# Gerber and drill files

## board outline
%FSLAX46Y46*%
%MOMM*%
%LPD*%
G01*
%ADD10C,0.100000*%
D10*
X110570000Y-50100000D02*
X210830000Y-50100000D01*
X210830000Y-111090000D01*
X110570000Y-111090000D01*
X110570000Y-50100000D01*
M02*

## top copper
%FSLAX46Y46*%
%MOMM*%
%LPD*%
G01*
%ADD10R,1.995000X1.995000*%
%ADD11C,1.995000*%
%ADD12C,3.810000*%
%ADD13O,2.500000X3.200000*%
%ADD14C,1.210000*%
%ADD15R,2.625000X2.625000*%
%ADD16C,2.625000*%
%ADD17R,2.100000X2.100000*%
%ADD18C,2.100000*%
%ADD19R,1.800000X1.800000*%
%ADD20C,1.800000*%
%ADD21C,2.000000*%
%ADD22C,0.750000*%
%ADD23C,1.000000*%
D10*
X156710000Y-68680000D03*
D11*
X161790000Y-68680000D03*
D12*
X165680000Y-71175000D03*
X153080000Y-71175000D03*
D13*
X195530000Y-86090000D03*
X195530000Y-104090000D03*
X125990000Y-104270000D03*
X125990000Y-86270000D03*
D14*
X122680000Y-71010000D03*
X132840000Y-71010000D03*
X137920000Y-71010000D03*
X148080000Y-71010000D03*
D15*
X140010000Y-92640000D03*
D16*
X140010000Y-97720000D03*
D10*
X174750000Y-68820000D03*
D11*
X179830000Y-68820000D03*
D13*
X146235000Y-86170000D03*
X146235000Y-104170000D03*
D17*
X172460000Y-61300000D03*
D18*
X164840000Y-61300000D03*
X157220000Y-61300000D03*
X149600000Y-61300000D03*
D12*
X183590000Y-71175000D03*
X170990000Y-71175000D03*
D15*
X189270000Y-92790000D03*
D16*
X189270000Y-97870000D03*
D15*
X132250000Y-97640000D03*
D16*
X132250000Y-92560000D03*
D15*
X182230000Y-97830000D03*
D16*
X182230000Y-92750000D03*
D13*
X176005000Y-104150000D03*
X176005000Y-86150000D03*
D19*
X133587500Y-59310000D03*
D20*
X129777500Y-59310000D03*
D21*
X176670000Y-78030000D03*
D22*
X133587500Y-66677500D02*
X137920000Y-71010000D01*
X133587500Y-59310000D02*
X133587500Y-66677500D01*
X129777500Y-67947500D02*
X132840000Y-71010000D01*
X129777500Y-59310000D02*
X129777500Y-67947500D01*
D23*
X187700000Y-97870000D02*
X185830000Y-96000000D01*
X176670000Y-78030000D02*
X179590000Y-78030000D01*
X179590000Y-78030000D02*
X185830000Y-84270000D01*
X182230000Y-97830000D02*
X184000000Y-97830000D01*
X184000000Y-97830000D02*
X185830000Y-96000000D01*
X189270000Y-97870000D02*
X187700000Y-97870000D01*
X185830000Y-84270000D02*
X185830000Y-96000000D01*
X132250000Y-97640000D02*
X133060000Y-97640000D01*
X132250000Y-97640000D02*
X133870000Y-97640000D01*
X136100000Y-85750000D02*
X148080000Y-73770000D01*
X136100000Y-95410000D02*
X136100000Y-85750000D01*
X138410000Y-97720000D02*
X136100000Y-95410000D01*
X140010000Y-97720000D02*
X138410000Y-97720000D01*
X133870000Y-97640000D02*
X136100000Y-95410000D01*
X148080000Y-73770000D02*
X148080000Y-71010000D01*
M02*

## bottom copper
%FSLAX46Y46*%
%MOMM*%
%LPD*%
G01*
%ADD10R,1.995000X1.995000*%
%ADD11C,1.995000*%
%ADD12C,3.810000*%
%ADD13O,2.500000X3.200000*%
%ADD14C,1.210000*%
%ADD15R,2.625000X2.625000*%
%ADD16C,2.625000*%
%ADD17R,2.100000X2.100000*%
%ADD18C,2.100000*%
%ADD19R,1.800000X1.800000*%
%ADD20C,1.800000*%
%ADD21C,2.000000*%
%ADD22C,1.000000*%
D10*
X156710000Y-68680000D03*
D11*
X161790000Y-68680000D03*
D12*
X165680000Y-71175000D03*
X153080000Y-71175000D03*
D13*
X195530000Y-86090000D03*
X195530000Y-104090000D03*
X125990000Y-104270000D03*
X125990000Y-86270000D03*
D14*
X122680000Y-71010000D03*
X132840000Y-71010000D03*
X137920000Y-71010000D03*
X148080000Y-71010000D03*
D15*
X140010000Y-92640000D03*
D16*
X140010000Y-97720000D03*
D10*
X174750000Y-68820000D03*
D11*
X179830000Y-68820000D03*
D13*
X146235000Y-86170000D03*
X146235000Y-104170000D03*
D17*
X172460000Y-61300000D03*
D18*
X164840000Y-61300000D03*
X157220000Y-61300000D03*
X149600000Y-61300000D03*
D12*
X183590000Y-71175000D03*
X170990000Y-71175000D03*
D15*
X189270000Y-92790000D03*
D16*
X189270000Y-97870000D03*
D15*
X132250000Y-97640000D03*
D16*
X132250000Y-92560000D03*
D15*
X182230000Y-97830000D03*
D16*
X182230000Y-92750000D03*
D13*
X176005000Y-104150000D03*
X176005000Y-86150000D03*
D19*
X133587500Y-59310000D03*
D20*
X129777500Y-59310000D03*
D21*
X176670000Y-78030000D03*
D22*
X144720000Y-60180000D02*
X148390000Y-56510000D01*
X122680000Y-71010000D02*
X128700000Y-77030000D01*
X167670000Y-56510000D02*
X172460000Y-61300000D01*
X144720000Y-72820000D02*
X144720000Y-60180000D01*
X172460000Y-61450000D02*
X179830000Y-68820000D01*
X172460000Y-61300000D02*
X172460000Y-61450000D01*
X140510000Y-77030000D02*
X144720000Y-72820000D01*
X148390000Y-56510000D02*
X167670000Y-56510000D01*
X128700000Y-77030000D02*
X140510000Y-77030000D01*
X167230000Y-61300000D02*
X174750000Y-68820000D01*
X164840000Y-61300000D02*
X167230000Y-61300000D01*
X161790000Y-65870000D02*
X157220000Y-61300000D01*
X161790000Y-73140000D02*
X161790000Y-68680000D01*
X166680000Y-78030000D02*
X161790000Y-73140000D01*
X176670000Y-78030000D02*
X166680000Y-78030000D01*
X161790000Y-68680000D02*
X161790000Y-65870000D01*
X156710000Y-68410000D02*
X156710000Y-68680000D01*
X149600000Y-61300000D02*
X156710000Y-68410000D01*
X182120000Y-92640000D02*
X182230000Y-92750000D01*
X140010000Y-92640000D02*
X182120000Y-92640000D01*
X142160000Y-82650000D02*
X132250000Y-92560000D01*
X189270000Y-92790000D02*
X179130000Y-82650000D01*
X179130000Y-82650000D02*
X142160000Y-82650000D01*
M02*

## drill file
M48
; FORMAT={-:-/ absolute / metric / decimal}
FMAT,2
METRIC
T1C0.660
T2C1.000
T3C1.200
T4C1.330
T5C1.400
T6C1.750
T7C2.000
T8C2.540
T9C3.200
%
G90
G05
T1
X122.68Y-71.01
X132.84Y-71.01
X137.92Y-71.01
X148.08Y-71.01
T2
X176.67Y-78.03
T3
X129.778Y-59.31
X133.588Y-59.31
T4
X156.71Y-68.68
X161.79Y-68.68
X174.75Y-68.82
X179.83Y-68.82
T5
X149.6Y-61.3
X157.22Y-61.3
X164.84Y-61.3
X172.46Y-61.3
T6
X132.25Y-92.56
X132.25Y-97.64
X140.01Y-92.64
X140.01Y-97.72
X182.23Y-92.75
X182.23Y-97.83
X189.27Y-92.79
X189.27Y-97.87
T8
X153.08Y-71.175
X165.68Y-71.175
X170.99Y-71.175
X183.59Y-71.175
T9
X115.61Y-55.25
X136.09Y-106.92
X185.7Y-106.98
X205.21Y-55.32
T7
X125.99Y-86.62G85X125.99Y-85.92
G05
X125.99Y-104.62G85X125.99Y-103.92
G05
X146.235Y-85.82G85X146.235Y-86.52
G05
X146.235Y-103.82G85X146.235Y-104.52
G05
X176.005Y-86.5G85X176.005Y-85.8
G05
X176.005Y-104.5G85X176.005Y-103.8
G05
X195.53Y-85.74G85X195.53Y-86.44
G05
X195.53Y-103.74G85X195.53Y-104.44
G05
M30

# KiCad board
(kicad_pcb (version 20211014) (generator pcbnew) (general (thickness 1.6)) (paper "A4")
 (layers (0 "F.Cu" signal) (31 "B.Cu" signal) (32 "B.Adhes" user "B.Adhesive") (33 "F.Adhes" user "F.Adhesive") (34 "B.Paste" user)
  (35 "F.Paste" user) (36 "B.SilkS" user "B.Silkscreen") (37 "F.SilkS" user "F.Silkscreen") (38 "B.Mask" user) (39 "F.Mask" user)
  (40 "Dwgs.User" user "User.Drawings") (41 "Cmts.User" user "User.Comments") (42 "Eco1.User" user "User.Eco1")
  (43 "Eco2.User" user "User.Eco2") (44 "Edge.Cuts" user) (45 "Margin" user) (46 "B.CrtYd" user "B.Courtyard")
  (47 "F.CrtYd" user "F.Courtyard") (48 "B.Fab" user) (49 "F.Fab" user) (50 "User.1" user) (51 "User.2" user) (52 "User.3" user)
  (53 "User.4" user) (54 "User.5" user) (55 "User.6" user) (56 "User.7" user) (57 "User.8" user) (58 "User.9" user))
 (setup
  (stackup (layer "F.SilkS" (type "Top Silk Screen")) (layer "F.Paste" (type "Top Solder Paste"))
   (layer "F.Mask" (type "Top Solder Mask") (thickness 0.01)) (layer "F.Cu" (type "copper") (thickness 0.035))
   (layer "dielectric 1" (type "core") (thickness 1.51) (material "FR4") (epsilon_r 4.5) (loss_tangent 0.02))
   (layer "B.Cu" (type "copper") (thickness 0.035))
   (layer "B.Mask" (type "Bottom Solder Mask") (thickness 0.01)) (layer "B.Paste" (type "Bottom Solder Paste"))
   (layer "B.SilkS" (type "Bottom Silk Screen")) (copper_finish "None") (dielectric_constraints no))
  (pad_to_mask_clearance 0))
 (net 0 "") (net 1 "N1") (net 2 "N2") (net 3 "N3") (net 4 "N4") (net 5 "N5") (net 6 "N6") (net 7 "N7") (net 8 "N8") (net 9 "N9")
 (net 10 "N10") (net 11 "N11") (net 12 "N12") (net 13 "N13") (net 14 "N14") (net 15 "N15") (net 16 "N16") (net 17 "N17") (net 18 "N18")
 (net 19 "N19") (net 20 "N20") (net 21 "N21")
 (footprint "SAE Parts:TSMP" (layer "F.Cu") (at 156.71 68.68)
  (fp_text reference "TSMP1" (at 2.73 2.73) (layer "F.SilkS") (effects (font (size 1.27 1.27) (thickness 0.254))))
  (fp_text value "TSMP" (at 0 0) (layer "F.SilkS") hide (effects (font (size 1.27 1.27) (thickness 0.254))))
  (pad "1" thru_hole rect (at 0 0) (size 1.995 1.995) (drill 1.33) (layers *.Cu *.Mask) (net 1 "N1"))
  (pad "2" thru_hole circle (at 5.08 0) (size 1.995 1.995) (drill 1.33) (layers *.Cu *.Mask) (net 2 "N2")))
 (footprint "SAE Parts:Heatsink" (layer "F.Cu") (at 165.68 71.175 180)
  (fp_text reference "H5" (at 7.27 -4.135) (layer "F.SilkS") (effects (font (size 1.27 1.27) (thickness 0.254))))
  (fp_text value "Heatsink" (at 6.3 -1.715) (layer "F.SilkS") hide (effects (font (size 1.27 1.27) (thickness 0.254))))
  (pad "1" thru_hole circle (at 0 0 180) (size 3.81 3.81) (drill 2.54) (layers *.Cu *.Mask) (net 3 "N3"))
  (pad "2" thru_hole circle (at 12.6 0 180) (size 3.81 3.81) (drill 2.54) (layers *.Cu *.Mask) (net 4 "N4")))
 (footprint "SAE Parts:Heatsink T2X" (layer "F.Cu") (at 201.405 95.19 -90)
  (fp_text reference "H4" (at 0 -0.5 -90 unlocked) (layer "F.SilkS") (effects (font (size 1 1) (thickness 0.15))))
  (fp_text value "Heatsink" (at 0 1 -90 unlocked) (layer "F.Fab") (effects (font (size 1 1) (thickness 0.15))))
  (pad "1" thru_hole oval (at -9.1 5.875 270) (size 3.2 2.5) (drill oval 2.7 2) (layers *.Cu *.Mask) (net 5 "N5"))
  (pad "2" thru_hole oval (at 8.9 5.875 270) (size 3.2 2.5) (drill oval 2.7 2) (layers *.Cu *.Mask) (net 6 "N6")))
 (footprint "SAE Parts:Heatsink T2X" (layer "F.Cu") (at 120.115 95.17 90)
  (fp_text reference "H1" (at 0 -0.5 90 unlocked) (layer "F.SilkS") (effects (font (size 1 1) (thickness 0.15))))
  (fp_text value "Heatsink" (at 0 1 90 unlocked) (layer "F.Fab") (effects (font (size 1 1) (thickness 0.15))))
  (pad "1" thru_hole oval (at -9.1 5.875 90) (size 3.2 2.5) (drill oval 2.7 2) (layers *.Cu *.Mask) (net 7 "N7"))
  (pad "2" thru_hole oval (at 8.9 5.875 90) (size 3.2 2.5) (drill oval 2.7 2) (layers *.Cu *.Mask) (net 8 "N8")))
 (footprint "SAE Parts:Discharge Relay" (layer "F.Cu") (at 122.68 71.01)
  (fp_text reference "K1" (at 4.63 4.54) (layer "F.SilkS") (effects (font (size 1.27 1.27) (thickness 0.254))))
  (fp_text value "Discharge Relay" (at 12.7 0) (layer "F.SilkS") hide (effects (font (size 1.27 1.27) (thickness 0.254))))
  (pad "1" thru_hole circle (at 0 0) (size 1.21 1.21) (drill 0.66) (layers *.Cu *.Mask) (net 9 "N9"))
  (pad "2" thru_hole circle (at 10.16 0) (size 1.21 1.21) (drill 0.66) (layers *.Cu *.Mask) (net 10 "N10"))
  (pad "3" thru_hole circle (at 15.24 0) (size 1.21 1.21) (drill 0.66) (layers *.Cu *.Mask) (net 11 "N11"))
  (pad "4" thru_hole circle (at 25.4 0) (size 1.21 1.21) (drill 0.66) (layers *.Cu *.Mask) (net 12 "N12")))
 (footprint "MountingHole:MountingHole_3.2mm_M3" (layer "F.Cu") (at 185.7 106.98)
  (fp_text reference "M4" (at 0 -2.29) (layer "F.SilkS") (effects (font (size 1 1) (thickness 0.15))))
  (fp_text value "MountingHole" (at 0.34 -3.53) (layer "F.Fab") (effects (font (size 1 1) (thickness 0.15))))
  (pad "" np_thru_hole circle (at 0 0) (size 3.2 3.2) (drill 3.2) (layers *.Cu *.Mask)))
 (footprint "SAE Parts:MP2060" (layer "F.Cu") (at 140.01 92.64 -90)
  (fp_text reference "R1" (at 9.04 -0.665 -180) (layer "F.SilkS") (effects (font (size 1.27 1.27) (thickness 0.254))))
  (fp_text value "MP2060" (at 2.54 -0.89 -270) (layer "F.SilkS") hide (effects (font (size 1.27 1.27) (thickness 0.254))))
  (pad "1" thru_hole rect (at 0 0 270) (size 2.625 2.625) (drill 1.75) (layers *.Cu *.Mask) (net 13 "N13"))
  (pad "2" thru_hole circle (at 5.08 0 270) (size 2.625 2.625) (drill 1.75) (layers *.Cu *.Mask) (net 12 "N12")))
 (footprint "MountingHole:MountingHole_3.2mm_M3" (layer "F.Cu") (at 115.61 55.25)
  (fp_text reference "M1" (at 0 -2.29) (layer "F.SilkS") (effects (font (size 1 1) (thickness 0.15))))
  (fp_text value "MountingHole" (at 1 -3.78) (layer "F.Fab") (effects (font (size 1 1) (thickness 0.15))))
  (pad "" np_thru_hole circle (at 0 0) (size 3.2 3.2) (drill 3.2) (layers *.Cu *.Mask)))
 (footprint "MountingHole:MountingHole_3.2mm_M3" (layer "F.Cu") (at 136.09 106.92)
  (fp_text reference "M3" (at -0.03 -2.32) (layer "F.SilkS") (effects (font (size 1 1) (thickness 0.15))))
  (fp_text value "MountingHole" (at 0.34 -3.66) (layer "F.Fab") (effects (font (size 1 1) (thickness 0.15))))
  (pad "" np_thru_hole circle (at 0 0) (size 3.2 3.2) (drill 3.2) (layers *.Cu *.Mask)))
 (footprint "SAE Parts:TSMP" (layer "F.Cu") (at 174.75 68.82)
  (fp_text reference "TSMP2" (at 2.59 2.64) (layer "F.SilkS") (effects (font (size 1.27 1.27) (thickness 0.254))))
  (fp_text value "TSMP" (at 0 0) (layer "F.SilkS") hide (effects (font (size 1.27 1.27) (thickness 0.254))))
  (pad "1" thru_hole rect (at 0 0) (size 1.995 1.995) (drill 1.33) (layers *.Cu *.Mask) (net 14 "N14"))
  (pad "2" thru_hole circle (at 5.08 0) (size 1.995 1.995) (drill 1.33) (layers *.Cu *.Mask) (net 9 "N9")))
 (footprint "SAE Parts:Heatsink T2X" (layer "F.Cu") (at 152.11 95.27 -90)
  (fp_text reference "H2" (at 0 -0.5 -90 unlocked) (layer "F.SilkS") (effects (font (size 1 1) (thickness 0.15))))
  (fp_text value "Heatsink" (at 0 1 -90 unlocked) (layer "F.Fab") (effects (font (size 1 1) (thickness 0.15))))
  (pad "1" thru_hole oval (at -9.1 5.875 270) (size 3.2 2.5) (drill oval 2.7 2) (layers *.Cu *.Mask) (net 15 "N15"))
  (pad "2" thru_hole oval (at 8.9 5.875 270) (size 3.2 2.5) (drill oval 2.7 2) (layers *.Cu *.Mask) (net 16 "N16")))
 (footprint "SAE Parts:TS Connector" (layer "F.Cu") (at 172.46 61.3 180)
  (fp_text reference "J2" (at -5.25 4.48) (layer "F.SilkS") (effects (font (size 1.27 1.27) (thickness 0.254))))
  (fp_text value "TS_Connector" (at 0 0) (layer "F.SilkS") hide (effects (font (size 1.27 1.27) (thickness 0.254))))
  (pad "1" thru_hole rect (at 0 0 180) (size 2.1 2.1) (drill 1.4) (layers *.Cu *.Mask) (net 9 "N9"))
  (pad "2" thru_hole circle (at 7.62 0 180) (size 2.1 2.1) (drill 1.4) (layers *.Cu *.Mask) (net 14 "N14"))
  (pad "3" thru_hole circle (at 15.24 0 180) (size 2.1 2.1) (drill 1.4) (layers *.Cu *.Mask) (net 2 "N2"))
  (pad "4" thru_hole circle (at 22.86 0 180) (size 2.1 2.1) (drill 1.4) (layers *.Cu *.Mask) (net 1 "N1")))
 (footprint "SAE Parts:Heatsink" (layer "F.Cu") (at 183.59 71.175 180)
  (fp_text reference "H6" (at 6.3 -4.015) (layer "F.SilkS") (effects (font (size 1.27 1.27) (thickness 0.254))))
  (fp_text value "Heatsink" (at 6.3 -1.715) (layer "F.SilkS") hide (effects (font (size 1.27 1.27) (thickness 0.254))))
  (pad "1" thru_hole circle (at 0 0 180) (size 3.81 3.81) (drill 2.54) (layers *.Cu *.Mask) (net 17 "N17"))
  (pad "2" thru_hole circle (at 12.6 0 180) (size 3.81 3.81) (drill 2.54) (layers *.Cu *.Mask) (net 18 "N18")))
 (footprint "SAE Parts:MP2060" (layer "F.Cu") (at 189.27 92.79 -90)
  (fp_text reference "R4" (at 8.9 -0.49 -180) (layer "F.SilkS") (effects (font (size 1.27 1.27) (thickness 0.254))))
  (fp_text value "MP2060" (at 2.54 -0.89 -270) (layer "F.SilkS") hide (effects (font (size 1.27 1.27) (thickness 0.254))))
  (pad "1" thru_hole rect (at 0 0 270) (size 2.625 2.625) (drill 1.75) (layers *.Cu *.Mask) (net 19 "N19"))
  (pad "2" thru_hole circle (at 5.08 0 270) (size 2.625 2.625) (drill 1.75) (layers *.Cu *.Mask) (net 2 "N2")))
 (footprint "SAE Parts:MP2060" (layer "F.Cu") (at 132.25 97.64 90)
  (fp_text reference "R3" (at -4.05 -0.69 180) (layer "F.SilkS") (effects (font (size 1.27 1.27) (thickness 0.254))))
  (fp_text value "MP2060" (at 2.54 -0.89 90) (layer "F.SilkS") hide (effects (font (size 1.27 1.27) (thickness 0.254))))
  (pad "1" thru_hole rect (at 0 0 90) (size 2.625 2.625) (drill 1.75) (layers *.Cu *.Mask) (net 12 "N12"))
  (pad "2" thru_hole circle (at 5.08 0 90) (size 2.625 2.625) (drill 1.75) (layers *.Cu *.Mask) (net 19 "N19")))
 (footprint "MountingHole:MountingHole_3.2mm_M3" (layer "F.Cu") (at 205.21 55.32)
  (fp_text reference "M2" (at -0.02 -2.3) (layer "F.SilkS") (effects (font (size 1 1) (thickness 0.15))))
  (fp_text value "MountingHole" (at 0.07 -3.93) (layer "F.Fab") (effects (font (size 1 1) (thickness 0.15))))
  (pad "" np_thru_hole circle (at 0 0) (size 3.2 3.2) (drill 3.2) (layers *.Cu *.Mask)))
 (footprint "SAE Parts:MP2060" (layer "F.Cu") (at 182.23 97.83 90)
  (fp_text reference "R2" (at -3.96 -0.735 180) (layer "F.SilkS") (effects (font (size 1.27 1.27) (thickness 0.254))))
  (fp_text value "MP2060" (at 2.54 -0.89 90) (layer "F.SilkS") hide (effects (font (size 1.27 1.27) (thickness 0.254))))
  (pad "1" thru_hole rect (at 0 0 90) (size 2.625 2.625) (drill 1.75) (layers *.Cu *.Mask) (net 2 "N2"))
  (pad "2" thru_hole circle (at 5.08 0 90) (size 2.625 2.625) (drill 1.75) (layers *.Cu *.Mask) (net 13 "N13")))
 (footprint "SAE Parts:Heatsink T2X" (layer "F.Cu") (at 170.13 95.05 90)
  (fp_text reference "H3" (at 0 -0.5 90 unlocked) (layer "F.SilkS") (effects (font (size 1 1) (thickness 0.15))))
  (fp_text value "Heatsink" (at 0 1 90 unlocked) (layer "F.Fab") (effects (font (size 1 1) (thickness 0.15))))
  (pad "1" thru_hole oval (at -9.1 5.875 90) (size 3.2 2.5) (drill oval 2.7 2) (layers *.Cu *.Mask) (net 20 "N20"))
  (pad "2" thru_hole oval (at 8.9 5.875 90) (size 3.2 2.5) (drill oval 2.7 2) (layers *.Cu *.Mask) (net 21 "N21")))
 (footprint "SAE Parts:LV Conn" (layer "F.Cu") (at 133.5875 59.31 180)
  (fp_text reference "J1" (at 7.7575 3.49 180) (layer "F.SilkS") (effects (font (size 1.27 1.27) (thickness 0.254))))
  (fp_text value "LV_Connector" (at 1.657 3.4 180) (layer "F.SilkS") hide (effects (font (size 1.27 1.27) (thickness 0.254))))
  (pad "1" thru_hole rect (at 0 0 180) (size 1.8 1.8) (drill 1.2) (layers *.Cu *.Mask) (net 11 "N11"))
  (pad "2" thru_hole circle (at 3.81 0 180) (size 1.8 1.8) (drill 1.2) (layers *.Cu *.Mask) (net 10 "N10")))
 (gr_rect (start 110.57 50.1) (end 210.83 111.09) (layer "Edge.Cuts") (width 0.1) (fill none))
 (segment (start 133.5875 66.6775) (end 137.92 71.01) (width 0.75) (layer "F.Cu") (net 11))
 (segment (start 133.5875 59.31) (end 133.5875 66.6775) (width 0.75) (layer "F.Cu") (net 11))
 (segment (start 129.7775 67.9475) (end 132.84 71.01) (width 0.75) (layer "F.Cu") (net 10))
 (segment (start 129.7775 59.31) (end 129.7775 67.9475) (width 0.75) (layer "F.Cu") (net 10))
 (segment (start 144.72 60.18) (end 148.39 56.51) (width 1) (layer "B.Cu") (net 9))
 (segment (start 122.68 71.01) (end 128.7 77.03) (width 1) (layer "B.Cu") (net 9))
 (segment (start 167.67 56.51) (end 172.46 61.3) (width 1) (layer "B.Cu") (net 9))
 (segment (start 144.72 72.82) (end 144.72 60.18) (width 1) (layer "B.Cu") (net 9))
 (segment (start 172.46 61.45) (end 179.83 68.82) (width 1) (layer "B.Cu") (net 9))
 (segment (start 172.46 61.3) (end 172.46 61.45) (width 1) (layer "B.Cu") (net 9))
 (segment (start 140.51 77.03) (end 144.72 72.82) (width 1) (layer "B.Cu") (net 9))
 (segment (start 148.39 56.51) (end 167.67 56.51) (width 1) (layer "B.Cu") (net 9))
 (segment (start 128.7 77.03) (end 140.51 77.03) (width 1) (layer "B.Cu") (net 9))
 (segment (start 167.23 61.3) (end 174.75 68.82) (width 1) (layer "B.Cu") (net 14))
 (segment (start 164.84 61.3) (end 167.23 61.3) (width 1) (layer "B.Cu") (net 14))
 (segment (start 187.7 97.87) (end 185.83 96) (width 1) (layer "F.Cu") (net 2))
 (segment (start 176.67 78.03) (end 179.59 78.03) (width 1) (layer "F.Cu") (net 2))
 (segment (start 179.59 78.03) (end 185.83 84.27) (width 1) (layer "F.Cu") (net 2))
 (segment (start 182.23 97.83) (end 184 97.83) (width 1) (layer "F.Cu") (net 2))
 (segment (start 184 97.83) (end 185.83 96) (width 1) (layer "F.Cu") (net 2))
 (segment (start 189.27 97.87) (end 187.7 97.87) (width 1) (layer "F.Cu") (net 2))
 (segment (start 185.83 84.27) (end 185.83 96) (width 1) (layer "F.Cu") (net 2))
 (via (at 176.67 78.03) (size 2) (drill 1) (layers "F.Cu" "B.Cu") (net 2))
 (segment (start 161.79 65.87) (end 157.22 61.3) (width 1) (layer "B.Cu") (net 2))
 (segment (start 161.79 73.14) (end 161.79 68.68) (width 1) (layer "B.Cu") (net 2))
 (segment (start 166.68 78.03) (end 161.79 73.14) (width 1) (layer "B.Cu") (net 2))
 (segment (start 176.67 78.03) (end 166.68 78.03) (width 1) (layer "B.Cu") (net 2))
 (segment (start 161.79 68.68) (end 161.79 65.87) (width 1) (layer "B.Cu") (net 2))
 (segment (start 156.71 68.41) (end 156.71 68.68) (width 1) (layer "B.Cu") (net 1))
 (segment (start 149.6 61.3) (end 156.71 68.41) (width 1) (layer "B.Cu") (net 1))
 (segment (start 132.25 97.64) (end 133.06 97.64) (width 1) (layer "F.Cu") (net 12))
 (segment (start 132.25 97.64) (end 133.87 97.64) (width 1) (layer "F.Cu") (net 12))
 (segment (start 136.1 85.75) (end 148.08 73.77) (width 1) (layer "F.Cu") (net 12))
 (segment (start 136.1 95.41) (end 136.1 85.75) (width 1) (layer "F.Cu") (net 12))
 (segment (start 138.41 97.72) (end 136.1 95.41) (width 1) (layer "F.Cu") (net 12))
 (segment (start 140.01 97.72) (end 138.41 97.72) (width 1) (layer "F.Cu") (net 12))
 (segment (start 133.87 97.64) (end 136.1 95.41) (width 1) (layer "F.Cu") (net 12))
 (segment (start 148.08 73.77) (end 148.08 71.01) (width 1) (layer "F.Cu") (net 12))
 (segment (start 182.12 92.64) (end 182.23 92.75) (width 1) (layer "B.Cu") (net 13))
 (segment (start 140.01 92.64) (end 182.12 92.64) (width 1) (layer "B.Cu") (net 13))
 (segment (start 142.16 82.65) (end 132.25 92.56) (width 1) (layer "B.Cu") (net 19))
 (segment (start 189.27 92.79) (end 179.13 82.65) (width 1) (layer "B.Cu") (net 19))
 (segment (start 179.13 82.65) (end 142.16 82.65) (width 1) (layer "B.Cu") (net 19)))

